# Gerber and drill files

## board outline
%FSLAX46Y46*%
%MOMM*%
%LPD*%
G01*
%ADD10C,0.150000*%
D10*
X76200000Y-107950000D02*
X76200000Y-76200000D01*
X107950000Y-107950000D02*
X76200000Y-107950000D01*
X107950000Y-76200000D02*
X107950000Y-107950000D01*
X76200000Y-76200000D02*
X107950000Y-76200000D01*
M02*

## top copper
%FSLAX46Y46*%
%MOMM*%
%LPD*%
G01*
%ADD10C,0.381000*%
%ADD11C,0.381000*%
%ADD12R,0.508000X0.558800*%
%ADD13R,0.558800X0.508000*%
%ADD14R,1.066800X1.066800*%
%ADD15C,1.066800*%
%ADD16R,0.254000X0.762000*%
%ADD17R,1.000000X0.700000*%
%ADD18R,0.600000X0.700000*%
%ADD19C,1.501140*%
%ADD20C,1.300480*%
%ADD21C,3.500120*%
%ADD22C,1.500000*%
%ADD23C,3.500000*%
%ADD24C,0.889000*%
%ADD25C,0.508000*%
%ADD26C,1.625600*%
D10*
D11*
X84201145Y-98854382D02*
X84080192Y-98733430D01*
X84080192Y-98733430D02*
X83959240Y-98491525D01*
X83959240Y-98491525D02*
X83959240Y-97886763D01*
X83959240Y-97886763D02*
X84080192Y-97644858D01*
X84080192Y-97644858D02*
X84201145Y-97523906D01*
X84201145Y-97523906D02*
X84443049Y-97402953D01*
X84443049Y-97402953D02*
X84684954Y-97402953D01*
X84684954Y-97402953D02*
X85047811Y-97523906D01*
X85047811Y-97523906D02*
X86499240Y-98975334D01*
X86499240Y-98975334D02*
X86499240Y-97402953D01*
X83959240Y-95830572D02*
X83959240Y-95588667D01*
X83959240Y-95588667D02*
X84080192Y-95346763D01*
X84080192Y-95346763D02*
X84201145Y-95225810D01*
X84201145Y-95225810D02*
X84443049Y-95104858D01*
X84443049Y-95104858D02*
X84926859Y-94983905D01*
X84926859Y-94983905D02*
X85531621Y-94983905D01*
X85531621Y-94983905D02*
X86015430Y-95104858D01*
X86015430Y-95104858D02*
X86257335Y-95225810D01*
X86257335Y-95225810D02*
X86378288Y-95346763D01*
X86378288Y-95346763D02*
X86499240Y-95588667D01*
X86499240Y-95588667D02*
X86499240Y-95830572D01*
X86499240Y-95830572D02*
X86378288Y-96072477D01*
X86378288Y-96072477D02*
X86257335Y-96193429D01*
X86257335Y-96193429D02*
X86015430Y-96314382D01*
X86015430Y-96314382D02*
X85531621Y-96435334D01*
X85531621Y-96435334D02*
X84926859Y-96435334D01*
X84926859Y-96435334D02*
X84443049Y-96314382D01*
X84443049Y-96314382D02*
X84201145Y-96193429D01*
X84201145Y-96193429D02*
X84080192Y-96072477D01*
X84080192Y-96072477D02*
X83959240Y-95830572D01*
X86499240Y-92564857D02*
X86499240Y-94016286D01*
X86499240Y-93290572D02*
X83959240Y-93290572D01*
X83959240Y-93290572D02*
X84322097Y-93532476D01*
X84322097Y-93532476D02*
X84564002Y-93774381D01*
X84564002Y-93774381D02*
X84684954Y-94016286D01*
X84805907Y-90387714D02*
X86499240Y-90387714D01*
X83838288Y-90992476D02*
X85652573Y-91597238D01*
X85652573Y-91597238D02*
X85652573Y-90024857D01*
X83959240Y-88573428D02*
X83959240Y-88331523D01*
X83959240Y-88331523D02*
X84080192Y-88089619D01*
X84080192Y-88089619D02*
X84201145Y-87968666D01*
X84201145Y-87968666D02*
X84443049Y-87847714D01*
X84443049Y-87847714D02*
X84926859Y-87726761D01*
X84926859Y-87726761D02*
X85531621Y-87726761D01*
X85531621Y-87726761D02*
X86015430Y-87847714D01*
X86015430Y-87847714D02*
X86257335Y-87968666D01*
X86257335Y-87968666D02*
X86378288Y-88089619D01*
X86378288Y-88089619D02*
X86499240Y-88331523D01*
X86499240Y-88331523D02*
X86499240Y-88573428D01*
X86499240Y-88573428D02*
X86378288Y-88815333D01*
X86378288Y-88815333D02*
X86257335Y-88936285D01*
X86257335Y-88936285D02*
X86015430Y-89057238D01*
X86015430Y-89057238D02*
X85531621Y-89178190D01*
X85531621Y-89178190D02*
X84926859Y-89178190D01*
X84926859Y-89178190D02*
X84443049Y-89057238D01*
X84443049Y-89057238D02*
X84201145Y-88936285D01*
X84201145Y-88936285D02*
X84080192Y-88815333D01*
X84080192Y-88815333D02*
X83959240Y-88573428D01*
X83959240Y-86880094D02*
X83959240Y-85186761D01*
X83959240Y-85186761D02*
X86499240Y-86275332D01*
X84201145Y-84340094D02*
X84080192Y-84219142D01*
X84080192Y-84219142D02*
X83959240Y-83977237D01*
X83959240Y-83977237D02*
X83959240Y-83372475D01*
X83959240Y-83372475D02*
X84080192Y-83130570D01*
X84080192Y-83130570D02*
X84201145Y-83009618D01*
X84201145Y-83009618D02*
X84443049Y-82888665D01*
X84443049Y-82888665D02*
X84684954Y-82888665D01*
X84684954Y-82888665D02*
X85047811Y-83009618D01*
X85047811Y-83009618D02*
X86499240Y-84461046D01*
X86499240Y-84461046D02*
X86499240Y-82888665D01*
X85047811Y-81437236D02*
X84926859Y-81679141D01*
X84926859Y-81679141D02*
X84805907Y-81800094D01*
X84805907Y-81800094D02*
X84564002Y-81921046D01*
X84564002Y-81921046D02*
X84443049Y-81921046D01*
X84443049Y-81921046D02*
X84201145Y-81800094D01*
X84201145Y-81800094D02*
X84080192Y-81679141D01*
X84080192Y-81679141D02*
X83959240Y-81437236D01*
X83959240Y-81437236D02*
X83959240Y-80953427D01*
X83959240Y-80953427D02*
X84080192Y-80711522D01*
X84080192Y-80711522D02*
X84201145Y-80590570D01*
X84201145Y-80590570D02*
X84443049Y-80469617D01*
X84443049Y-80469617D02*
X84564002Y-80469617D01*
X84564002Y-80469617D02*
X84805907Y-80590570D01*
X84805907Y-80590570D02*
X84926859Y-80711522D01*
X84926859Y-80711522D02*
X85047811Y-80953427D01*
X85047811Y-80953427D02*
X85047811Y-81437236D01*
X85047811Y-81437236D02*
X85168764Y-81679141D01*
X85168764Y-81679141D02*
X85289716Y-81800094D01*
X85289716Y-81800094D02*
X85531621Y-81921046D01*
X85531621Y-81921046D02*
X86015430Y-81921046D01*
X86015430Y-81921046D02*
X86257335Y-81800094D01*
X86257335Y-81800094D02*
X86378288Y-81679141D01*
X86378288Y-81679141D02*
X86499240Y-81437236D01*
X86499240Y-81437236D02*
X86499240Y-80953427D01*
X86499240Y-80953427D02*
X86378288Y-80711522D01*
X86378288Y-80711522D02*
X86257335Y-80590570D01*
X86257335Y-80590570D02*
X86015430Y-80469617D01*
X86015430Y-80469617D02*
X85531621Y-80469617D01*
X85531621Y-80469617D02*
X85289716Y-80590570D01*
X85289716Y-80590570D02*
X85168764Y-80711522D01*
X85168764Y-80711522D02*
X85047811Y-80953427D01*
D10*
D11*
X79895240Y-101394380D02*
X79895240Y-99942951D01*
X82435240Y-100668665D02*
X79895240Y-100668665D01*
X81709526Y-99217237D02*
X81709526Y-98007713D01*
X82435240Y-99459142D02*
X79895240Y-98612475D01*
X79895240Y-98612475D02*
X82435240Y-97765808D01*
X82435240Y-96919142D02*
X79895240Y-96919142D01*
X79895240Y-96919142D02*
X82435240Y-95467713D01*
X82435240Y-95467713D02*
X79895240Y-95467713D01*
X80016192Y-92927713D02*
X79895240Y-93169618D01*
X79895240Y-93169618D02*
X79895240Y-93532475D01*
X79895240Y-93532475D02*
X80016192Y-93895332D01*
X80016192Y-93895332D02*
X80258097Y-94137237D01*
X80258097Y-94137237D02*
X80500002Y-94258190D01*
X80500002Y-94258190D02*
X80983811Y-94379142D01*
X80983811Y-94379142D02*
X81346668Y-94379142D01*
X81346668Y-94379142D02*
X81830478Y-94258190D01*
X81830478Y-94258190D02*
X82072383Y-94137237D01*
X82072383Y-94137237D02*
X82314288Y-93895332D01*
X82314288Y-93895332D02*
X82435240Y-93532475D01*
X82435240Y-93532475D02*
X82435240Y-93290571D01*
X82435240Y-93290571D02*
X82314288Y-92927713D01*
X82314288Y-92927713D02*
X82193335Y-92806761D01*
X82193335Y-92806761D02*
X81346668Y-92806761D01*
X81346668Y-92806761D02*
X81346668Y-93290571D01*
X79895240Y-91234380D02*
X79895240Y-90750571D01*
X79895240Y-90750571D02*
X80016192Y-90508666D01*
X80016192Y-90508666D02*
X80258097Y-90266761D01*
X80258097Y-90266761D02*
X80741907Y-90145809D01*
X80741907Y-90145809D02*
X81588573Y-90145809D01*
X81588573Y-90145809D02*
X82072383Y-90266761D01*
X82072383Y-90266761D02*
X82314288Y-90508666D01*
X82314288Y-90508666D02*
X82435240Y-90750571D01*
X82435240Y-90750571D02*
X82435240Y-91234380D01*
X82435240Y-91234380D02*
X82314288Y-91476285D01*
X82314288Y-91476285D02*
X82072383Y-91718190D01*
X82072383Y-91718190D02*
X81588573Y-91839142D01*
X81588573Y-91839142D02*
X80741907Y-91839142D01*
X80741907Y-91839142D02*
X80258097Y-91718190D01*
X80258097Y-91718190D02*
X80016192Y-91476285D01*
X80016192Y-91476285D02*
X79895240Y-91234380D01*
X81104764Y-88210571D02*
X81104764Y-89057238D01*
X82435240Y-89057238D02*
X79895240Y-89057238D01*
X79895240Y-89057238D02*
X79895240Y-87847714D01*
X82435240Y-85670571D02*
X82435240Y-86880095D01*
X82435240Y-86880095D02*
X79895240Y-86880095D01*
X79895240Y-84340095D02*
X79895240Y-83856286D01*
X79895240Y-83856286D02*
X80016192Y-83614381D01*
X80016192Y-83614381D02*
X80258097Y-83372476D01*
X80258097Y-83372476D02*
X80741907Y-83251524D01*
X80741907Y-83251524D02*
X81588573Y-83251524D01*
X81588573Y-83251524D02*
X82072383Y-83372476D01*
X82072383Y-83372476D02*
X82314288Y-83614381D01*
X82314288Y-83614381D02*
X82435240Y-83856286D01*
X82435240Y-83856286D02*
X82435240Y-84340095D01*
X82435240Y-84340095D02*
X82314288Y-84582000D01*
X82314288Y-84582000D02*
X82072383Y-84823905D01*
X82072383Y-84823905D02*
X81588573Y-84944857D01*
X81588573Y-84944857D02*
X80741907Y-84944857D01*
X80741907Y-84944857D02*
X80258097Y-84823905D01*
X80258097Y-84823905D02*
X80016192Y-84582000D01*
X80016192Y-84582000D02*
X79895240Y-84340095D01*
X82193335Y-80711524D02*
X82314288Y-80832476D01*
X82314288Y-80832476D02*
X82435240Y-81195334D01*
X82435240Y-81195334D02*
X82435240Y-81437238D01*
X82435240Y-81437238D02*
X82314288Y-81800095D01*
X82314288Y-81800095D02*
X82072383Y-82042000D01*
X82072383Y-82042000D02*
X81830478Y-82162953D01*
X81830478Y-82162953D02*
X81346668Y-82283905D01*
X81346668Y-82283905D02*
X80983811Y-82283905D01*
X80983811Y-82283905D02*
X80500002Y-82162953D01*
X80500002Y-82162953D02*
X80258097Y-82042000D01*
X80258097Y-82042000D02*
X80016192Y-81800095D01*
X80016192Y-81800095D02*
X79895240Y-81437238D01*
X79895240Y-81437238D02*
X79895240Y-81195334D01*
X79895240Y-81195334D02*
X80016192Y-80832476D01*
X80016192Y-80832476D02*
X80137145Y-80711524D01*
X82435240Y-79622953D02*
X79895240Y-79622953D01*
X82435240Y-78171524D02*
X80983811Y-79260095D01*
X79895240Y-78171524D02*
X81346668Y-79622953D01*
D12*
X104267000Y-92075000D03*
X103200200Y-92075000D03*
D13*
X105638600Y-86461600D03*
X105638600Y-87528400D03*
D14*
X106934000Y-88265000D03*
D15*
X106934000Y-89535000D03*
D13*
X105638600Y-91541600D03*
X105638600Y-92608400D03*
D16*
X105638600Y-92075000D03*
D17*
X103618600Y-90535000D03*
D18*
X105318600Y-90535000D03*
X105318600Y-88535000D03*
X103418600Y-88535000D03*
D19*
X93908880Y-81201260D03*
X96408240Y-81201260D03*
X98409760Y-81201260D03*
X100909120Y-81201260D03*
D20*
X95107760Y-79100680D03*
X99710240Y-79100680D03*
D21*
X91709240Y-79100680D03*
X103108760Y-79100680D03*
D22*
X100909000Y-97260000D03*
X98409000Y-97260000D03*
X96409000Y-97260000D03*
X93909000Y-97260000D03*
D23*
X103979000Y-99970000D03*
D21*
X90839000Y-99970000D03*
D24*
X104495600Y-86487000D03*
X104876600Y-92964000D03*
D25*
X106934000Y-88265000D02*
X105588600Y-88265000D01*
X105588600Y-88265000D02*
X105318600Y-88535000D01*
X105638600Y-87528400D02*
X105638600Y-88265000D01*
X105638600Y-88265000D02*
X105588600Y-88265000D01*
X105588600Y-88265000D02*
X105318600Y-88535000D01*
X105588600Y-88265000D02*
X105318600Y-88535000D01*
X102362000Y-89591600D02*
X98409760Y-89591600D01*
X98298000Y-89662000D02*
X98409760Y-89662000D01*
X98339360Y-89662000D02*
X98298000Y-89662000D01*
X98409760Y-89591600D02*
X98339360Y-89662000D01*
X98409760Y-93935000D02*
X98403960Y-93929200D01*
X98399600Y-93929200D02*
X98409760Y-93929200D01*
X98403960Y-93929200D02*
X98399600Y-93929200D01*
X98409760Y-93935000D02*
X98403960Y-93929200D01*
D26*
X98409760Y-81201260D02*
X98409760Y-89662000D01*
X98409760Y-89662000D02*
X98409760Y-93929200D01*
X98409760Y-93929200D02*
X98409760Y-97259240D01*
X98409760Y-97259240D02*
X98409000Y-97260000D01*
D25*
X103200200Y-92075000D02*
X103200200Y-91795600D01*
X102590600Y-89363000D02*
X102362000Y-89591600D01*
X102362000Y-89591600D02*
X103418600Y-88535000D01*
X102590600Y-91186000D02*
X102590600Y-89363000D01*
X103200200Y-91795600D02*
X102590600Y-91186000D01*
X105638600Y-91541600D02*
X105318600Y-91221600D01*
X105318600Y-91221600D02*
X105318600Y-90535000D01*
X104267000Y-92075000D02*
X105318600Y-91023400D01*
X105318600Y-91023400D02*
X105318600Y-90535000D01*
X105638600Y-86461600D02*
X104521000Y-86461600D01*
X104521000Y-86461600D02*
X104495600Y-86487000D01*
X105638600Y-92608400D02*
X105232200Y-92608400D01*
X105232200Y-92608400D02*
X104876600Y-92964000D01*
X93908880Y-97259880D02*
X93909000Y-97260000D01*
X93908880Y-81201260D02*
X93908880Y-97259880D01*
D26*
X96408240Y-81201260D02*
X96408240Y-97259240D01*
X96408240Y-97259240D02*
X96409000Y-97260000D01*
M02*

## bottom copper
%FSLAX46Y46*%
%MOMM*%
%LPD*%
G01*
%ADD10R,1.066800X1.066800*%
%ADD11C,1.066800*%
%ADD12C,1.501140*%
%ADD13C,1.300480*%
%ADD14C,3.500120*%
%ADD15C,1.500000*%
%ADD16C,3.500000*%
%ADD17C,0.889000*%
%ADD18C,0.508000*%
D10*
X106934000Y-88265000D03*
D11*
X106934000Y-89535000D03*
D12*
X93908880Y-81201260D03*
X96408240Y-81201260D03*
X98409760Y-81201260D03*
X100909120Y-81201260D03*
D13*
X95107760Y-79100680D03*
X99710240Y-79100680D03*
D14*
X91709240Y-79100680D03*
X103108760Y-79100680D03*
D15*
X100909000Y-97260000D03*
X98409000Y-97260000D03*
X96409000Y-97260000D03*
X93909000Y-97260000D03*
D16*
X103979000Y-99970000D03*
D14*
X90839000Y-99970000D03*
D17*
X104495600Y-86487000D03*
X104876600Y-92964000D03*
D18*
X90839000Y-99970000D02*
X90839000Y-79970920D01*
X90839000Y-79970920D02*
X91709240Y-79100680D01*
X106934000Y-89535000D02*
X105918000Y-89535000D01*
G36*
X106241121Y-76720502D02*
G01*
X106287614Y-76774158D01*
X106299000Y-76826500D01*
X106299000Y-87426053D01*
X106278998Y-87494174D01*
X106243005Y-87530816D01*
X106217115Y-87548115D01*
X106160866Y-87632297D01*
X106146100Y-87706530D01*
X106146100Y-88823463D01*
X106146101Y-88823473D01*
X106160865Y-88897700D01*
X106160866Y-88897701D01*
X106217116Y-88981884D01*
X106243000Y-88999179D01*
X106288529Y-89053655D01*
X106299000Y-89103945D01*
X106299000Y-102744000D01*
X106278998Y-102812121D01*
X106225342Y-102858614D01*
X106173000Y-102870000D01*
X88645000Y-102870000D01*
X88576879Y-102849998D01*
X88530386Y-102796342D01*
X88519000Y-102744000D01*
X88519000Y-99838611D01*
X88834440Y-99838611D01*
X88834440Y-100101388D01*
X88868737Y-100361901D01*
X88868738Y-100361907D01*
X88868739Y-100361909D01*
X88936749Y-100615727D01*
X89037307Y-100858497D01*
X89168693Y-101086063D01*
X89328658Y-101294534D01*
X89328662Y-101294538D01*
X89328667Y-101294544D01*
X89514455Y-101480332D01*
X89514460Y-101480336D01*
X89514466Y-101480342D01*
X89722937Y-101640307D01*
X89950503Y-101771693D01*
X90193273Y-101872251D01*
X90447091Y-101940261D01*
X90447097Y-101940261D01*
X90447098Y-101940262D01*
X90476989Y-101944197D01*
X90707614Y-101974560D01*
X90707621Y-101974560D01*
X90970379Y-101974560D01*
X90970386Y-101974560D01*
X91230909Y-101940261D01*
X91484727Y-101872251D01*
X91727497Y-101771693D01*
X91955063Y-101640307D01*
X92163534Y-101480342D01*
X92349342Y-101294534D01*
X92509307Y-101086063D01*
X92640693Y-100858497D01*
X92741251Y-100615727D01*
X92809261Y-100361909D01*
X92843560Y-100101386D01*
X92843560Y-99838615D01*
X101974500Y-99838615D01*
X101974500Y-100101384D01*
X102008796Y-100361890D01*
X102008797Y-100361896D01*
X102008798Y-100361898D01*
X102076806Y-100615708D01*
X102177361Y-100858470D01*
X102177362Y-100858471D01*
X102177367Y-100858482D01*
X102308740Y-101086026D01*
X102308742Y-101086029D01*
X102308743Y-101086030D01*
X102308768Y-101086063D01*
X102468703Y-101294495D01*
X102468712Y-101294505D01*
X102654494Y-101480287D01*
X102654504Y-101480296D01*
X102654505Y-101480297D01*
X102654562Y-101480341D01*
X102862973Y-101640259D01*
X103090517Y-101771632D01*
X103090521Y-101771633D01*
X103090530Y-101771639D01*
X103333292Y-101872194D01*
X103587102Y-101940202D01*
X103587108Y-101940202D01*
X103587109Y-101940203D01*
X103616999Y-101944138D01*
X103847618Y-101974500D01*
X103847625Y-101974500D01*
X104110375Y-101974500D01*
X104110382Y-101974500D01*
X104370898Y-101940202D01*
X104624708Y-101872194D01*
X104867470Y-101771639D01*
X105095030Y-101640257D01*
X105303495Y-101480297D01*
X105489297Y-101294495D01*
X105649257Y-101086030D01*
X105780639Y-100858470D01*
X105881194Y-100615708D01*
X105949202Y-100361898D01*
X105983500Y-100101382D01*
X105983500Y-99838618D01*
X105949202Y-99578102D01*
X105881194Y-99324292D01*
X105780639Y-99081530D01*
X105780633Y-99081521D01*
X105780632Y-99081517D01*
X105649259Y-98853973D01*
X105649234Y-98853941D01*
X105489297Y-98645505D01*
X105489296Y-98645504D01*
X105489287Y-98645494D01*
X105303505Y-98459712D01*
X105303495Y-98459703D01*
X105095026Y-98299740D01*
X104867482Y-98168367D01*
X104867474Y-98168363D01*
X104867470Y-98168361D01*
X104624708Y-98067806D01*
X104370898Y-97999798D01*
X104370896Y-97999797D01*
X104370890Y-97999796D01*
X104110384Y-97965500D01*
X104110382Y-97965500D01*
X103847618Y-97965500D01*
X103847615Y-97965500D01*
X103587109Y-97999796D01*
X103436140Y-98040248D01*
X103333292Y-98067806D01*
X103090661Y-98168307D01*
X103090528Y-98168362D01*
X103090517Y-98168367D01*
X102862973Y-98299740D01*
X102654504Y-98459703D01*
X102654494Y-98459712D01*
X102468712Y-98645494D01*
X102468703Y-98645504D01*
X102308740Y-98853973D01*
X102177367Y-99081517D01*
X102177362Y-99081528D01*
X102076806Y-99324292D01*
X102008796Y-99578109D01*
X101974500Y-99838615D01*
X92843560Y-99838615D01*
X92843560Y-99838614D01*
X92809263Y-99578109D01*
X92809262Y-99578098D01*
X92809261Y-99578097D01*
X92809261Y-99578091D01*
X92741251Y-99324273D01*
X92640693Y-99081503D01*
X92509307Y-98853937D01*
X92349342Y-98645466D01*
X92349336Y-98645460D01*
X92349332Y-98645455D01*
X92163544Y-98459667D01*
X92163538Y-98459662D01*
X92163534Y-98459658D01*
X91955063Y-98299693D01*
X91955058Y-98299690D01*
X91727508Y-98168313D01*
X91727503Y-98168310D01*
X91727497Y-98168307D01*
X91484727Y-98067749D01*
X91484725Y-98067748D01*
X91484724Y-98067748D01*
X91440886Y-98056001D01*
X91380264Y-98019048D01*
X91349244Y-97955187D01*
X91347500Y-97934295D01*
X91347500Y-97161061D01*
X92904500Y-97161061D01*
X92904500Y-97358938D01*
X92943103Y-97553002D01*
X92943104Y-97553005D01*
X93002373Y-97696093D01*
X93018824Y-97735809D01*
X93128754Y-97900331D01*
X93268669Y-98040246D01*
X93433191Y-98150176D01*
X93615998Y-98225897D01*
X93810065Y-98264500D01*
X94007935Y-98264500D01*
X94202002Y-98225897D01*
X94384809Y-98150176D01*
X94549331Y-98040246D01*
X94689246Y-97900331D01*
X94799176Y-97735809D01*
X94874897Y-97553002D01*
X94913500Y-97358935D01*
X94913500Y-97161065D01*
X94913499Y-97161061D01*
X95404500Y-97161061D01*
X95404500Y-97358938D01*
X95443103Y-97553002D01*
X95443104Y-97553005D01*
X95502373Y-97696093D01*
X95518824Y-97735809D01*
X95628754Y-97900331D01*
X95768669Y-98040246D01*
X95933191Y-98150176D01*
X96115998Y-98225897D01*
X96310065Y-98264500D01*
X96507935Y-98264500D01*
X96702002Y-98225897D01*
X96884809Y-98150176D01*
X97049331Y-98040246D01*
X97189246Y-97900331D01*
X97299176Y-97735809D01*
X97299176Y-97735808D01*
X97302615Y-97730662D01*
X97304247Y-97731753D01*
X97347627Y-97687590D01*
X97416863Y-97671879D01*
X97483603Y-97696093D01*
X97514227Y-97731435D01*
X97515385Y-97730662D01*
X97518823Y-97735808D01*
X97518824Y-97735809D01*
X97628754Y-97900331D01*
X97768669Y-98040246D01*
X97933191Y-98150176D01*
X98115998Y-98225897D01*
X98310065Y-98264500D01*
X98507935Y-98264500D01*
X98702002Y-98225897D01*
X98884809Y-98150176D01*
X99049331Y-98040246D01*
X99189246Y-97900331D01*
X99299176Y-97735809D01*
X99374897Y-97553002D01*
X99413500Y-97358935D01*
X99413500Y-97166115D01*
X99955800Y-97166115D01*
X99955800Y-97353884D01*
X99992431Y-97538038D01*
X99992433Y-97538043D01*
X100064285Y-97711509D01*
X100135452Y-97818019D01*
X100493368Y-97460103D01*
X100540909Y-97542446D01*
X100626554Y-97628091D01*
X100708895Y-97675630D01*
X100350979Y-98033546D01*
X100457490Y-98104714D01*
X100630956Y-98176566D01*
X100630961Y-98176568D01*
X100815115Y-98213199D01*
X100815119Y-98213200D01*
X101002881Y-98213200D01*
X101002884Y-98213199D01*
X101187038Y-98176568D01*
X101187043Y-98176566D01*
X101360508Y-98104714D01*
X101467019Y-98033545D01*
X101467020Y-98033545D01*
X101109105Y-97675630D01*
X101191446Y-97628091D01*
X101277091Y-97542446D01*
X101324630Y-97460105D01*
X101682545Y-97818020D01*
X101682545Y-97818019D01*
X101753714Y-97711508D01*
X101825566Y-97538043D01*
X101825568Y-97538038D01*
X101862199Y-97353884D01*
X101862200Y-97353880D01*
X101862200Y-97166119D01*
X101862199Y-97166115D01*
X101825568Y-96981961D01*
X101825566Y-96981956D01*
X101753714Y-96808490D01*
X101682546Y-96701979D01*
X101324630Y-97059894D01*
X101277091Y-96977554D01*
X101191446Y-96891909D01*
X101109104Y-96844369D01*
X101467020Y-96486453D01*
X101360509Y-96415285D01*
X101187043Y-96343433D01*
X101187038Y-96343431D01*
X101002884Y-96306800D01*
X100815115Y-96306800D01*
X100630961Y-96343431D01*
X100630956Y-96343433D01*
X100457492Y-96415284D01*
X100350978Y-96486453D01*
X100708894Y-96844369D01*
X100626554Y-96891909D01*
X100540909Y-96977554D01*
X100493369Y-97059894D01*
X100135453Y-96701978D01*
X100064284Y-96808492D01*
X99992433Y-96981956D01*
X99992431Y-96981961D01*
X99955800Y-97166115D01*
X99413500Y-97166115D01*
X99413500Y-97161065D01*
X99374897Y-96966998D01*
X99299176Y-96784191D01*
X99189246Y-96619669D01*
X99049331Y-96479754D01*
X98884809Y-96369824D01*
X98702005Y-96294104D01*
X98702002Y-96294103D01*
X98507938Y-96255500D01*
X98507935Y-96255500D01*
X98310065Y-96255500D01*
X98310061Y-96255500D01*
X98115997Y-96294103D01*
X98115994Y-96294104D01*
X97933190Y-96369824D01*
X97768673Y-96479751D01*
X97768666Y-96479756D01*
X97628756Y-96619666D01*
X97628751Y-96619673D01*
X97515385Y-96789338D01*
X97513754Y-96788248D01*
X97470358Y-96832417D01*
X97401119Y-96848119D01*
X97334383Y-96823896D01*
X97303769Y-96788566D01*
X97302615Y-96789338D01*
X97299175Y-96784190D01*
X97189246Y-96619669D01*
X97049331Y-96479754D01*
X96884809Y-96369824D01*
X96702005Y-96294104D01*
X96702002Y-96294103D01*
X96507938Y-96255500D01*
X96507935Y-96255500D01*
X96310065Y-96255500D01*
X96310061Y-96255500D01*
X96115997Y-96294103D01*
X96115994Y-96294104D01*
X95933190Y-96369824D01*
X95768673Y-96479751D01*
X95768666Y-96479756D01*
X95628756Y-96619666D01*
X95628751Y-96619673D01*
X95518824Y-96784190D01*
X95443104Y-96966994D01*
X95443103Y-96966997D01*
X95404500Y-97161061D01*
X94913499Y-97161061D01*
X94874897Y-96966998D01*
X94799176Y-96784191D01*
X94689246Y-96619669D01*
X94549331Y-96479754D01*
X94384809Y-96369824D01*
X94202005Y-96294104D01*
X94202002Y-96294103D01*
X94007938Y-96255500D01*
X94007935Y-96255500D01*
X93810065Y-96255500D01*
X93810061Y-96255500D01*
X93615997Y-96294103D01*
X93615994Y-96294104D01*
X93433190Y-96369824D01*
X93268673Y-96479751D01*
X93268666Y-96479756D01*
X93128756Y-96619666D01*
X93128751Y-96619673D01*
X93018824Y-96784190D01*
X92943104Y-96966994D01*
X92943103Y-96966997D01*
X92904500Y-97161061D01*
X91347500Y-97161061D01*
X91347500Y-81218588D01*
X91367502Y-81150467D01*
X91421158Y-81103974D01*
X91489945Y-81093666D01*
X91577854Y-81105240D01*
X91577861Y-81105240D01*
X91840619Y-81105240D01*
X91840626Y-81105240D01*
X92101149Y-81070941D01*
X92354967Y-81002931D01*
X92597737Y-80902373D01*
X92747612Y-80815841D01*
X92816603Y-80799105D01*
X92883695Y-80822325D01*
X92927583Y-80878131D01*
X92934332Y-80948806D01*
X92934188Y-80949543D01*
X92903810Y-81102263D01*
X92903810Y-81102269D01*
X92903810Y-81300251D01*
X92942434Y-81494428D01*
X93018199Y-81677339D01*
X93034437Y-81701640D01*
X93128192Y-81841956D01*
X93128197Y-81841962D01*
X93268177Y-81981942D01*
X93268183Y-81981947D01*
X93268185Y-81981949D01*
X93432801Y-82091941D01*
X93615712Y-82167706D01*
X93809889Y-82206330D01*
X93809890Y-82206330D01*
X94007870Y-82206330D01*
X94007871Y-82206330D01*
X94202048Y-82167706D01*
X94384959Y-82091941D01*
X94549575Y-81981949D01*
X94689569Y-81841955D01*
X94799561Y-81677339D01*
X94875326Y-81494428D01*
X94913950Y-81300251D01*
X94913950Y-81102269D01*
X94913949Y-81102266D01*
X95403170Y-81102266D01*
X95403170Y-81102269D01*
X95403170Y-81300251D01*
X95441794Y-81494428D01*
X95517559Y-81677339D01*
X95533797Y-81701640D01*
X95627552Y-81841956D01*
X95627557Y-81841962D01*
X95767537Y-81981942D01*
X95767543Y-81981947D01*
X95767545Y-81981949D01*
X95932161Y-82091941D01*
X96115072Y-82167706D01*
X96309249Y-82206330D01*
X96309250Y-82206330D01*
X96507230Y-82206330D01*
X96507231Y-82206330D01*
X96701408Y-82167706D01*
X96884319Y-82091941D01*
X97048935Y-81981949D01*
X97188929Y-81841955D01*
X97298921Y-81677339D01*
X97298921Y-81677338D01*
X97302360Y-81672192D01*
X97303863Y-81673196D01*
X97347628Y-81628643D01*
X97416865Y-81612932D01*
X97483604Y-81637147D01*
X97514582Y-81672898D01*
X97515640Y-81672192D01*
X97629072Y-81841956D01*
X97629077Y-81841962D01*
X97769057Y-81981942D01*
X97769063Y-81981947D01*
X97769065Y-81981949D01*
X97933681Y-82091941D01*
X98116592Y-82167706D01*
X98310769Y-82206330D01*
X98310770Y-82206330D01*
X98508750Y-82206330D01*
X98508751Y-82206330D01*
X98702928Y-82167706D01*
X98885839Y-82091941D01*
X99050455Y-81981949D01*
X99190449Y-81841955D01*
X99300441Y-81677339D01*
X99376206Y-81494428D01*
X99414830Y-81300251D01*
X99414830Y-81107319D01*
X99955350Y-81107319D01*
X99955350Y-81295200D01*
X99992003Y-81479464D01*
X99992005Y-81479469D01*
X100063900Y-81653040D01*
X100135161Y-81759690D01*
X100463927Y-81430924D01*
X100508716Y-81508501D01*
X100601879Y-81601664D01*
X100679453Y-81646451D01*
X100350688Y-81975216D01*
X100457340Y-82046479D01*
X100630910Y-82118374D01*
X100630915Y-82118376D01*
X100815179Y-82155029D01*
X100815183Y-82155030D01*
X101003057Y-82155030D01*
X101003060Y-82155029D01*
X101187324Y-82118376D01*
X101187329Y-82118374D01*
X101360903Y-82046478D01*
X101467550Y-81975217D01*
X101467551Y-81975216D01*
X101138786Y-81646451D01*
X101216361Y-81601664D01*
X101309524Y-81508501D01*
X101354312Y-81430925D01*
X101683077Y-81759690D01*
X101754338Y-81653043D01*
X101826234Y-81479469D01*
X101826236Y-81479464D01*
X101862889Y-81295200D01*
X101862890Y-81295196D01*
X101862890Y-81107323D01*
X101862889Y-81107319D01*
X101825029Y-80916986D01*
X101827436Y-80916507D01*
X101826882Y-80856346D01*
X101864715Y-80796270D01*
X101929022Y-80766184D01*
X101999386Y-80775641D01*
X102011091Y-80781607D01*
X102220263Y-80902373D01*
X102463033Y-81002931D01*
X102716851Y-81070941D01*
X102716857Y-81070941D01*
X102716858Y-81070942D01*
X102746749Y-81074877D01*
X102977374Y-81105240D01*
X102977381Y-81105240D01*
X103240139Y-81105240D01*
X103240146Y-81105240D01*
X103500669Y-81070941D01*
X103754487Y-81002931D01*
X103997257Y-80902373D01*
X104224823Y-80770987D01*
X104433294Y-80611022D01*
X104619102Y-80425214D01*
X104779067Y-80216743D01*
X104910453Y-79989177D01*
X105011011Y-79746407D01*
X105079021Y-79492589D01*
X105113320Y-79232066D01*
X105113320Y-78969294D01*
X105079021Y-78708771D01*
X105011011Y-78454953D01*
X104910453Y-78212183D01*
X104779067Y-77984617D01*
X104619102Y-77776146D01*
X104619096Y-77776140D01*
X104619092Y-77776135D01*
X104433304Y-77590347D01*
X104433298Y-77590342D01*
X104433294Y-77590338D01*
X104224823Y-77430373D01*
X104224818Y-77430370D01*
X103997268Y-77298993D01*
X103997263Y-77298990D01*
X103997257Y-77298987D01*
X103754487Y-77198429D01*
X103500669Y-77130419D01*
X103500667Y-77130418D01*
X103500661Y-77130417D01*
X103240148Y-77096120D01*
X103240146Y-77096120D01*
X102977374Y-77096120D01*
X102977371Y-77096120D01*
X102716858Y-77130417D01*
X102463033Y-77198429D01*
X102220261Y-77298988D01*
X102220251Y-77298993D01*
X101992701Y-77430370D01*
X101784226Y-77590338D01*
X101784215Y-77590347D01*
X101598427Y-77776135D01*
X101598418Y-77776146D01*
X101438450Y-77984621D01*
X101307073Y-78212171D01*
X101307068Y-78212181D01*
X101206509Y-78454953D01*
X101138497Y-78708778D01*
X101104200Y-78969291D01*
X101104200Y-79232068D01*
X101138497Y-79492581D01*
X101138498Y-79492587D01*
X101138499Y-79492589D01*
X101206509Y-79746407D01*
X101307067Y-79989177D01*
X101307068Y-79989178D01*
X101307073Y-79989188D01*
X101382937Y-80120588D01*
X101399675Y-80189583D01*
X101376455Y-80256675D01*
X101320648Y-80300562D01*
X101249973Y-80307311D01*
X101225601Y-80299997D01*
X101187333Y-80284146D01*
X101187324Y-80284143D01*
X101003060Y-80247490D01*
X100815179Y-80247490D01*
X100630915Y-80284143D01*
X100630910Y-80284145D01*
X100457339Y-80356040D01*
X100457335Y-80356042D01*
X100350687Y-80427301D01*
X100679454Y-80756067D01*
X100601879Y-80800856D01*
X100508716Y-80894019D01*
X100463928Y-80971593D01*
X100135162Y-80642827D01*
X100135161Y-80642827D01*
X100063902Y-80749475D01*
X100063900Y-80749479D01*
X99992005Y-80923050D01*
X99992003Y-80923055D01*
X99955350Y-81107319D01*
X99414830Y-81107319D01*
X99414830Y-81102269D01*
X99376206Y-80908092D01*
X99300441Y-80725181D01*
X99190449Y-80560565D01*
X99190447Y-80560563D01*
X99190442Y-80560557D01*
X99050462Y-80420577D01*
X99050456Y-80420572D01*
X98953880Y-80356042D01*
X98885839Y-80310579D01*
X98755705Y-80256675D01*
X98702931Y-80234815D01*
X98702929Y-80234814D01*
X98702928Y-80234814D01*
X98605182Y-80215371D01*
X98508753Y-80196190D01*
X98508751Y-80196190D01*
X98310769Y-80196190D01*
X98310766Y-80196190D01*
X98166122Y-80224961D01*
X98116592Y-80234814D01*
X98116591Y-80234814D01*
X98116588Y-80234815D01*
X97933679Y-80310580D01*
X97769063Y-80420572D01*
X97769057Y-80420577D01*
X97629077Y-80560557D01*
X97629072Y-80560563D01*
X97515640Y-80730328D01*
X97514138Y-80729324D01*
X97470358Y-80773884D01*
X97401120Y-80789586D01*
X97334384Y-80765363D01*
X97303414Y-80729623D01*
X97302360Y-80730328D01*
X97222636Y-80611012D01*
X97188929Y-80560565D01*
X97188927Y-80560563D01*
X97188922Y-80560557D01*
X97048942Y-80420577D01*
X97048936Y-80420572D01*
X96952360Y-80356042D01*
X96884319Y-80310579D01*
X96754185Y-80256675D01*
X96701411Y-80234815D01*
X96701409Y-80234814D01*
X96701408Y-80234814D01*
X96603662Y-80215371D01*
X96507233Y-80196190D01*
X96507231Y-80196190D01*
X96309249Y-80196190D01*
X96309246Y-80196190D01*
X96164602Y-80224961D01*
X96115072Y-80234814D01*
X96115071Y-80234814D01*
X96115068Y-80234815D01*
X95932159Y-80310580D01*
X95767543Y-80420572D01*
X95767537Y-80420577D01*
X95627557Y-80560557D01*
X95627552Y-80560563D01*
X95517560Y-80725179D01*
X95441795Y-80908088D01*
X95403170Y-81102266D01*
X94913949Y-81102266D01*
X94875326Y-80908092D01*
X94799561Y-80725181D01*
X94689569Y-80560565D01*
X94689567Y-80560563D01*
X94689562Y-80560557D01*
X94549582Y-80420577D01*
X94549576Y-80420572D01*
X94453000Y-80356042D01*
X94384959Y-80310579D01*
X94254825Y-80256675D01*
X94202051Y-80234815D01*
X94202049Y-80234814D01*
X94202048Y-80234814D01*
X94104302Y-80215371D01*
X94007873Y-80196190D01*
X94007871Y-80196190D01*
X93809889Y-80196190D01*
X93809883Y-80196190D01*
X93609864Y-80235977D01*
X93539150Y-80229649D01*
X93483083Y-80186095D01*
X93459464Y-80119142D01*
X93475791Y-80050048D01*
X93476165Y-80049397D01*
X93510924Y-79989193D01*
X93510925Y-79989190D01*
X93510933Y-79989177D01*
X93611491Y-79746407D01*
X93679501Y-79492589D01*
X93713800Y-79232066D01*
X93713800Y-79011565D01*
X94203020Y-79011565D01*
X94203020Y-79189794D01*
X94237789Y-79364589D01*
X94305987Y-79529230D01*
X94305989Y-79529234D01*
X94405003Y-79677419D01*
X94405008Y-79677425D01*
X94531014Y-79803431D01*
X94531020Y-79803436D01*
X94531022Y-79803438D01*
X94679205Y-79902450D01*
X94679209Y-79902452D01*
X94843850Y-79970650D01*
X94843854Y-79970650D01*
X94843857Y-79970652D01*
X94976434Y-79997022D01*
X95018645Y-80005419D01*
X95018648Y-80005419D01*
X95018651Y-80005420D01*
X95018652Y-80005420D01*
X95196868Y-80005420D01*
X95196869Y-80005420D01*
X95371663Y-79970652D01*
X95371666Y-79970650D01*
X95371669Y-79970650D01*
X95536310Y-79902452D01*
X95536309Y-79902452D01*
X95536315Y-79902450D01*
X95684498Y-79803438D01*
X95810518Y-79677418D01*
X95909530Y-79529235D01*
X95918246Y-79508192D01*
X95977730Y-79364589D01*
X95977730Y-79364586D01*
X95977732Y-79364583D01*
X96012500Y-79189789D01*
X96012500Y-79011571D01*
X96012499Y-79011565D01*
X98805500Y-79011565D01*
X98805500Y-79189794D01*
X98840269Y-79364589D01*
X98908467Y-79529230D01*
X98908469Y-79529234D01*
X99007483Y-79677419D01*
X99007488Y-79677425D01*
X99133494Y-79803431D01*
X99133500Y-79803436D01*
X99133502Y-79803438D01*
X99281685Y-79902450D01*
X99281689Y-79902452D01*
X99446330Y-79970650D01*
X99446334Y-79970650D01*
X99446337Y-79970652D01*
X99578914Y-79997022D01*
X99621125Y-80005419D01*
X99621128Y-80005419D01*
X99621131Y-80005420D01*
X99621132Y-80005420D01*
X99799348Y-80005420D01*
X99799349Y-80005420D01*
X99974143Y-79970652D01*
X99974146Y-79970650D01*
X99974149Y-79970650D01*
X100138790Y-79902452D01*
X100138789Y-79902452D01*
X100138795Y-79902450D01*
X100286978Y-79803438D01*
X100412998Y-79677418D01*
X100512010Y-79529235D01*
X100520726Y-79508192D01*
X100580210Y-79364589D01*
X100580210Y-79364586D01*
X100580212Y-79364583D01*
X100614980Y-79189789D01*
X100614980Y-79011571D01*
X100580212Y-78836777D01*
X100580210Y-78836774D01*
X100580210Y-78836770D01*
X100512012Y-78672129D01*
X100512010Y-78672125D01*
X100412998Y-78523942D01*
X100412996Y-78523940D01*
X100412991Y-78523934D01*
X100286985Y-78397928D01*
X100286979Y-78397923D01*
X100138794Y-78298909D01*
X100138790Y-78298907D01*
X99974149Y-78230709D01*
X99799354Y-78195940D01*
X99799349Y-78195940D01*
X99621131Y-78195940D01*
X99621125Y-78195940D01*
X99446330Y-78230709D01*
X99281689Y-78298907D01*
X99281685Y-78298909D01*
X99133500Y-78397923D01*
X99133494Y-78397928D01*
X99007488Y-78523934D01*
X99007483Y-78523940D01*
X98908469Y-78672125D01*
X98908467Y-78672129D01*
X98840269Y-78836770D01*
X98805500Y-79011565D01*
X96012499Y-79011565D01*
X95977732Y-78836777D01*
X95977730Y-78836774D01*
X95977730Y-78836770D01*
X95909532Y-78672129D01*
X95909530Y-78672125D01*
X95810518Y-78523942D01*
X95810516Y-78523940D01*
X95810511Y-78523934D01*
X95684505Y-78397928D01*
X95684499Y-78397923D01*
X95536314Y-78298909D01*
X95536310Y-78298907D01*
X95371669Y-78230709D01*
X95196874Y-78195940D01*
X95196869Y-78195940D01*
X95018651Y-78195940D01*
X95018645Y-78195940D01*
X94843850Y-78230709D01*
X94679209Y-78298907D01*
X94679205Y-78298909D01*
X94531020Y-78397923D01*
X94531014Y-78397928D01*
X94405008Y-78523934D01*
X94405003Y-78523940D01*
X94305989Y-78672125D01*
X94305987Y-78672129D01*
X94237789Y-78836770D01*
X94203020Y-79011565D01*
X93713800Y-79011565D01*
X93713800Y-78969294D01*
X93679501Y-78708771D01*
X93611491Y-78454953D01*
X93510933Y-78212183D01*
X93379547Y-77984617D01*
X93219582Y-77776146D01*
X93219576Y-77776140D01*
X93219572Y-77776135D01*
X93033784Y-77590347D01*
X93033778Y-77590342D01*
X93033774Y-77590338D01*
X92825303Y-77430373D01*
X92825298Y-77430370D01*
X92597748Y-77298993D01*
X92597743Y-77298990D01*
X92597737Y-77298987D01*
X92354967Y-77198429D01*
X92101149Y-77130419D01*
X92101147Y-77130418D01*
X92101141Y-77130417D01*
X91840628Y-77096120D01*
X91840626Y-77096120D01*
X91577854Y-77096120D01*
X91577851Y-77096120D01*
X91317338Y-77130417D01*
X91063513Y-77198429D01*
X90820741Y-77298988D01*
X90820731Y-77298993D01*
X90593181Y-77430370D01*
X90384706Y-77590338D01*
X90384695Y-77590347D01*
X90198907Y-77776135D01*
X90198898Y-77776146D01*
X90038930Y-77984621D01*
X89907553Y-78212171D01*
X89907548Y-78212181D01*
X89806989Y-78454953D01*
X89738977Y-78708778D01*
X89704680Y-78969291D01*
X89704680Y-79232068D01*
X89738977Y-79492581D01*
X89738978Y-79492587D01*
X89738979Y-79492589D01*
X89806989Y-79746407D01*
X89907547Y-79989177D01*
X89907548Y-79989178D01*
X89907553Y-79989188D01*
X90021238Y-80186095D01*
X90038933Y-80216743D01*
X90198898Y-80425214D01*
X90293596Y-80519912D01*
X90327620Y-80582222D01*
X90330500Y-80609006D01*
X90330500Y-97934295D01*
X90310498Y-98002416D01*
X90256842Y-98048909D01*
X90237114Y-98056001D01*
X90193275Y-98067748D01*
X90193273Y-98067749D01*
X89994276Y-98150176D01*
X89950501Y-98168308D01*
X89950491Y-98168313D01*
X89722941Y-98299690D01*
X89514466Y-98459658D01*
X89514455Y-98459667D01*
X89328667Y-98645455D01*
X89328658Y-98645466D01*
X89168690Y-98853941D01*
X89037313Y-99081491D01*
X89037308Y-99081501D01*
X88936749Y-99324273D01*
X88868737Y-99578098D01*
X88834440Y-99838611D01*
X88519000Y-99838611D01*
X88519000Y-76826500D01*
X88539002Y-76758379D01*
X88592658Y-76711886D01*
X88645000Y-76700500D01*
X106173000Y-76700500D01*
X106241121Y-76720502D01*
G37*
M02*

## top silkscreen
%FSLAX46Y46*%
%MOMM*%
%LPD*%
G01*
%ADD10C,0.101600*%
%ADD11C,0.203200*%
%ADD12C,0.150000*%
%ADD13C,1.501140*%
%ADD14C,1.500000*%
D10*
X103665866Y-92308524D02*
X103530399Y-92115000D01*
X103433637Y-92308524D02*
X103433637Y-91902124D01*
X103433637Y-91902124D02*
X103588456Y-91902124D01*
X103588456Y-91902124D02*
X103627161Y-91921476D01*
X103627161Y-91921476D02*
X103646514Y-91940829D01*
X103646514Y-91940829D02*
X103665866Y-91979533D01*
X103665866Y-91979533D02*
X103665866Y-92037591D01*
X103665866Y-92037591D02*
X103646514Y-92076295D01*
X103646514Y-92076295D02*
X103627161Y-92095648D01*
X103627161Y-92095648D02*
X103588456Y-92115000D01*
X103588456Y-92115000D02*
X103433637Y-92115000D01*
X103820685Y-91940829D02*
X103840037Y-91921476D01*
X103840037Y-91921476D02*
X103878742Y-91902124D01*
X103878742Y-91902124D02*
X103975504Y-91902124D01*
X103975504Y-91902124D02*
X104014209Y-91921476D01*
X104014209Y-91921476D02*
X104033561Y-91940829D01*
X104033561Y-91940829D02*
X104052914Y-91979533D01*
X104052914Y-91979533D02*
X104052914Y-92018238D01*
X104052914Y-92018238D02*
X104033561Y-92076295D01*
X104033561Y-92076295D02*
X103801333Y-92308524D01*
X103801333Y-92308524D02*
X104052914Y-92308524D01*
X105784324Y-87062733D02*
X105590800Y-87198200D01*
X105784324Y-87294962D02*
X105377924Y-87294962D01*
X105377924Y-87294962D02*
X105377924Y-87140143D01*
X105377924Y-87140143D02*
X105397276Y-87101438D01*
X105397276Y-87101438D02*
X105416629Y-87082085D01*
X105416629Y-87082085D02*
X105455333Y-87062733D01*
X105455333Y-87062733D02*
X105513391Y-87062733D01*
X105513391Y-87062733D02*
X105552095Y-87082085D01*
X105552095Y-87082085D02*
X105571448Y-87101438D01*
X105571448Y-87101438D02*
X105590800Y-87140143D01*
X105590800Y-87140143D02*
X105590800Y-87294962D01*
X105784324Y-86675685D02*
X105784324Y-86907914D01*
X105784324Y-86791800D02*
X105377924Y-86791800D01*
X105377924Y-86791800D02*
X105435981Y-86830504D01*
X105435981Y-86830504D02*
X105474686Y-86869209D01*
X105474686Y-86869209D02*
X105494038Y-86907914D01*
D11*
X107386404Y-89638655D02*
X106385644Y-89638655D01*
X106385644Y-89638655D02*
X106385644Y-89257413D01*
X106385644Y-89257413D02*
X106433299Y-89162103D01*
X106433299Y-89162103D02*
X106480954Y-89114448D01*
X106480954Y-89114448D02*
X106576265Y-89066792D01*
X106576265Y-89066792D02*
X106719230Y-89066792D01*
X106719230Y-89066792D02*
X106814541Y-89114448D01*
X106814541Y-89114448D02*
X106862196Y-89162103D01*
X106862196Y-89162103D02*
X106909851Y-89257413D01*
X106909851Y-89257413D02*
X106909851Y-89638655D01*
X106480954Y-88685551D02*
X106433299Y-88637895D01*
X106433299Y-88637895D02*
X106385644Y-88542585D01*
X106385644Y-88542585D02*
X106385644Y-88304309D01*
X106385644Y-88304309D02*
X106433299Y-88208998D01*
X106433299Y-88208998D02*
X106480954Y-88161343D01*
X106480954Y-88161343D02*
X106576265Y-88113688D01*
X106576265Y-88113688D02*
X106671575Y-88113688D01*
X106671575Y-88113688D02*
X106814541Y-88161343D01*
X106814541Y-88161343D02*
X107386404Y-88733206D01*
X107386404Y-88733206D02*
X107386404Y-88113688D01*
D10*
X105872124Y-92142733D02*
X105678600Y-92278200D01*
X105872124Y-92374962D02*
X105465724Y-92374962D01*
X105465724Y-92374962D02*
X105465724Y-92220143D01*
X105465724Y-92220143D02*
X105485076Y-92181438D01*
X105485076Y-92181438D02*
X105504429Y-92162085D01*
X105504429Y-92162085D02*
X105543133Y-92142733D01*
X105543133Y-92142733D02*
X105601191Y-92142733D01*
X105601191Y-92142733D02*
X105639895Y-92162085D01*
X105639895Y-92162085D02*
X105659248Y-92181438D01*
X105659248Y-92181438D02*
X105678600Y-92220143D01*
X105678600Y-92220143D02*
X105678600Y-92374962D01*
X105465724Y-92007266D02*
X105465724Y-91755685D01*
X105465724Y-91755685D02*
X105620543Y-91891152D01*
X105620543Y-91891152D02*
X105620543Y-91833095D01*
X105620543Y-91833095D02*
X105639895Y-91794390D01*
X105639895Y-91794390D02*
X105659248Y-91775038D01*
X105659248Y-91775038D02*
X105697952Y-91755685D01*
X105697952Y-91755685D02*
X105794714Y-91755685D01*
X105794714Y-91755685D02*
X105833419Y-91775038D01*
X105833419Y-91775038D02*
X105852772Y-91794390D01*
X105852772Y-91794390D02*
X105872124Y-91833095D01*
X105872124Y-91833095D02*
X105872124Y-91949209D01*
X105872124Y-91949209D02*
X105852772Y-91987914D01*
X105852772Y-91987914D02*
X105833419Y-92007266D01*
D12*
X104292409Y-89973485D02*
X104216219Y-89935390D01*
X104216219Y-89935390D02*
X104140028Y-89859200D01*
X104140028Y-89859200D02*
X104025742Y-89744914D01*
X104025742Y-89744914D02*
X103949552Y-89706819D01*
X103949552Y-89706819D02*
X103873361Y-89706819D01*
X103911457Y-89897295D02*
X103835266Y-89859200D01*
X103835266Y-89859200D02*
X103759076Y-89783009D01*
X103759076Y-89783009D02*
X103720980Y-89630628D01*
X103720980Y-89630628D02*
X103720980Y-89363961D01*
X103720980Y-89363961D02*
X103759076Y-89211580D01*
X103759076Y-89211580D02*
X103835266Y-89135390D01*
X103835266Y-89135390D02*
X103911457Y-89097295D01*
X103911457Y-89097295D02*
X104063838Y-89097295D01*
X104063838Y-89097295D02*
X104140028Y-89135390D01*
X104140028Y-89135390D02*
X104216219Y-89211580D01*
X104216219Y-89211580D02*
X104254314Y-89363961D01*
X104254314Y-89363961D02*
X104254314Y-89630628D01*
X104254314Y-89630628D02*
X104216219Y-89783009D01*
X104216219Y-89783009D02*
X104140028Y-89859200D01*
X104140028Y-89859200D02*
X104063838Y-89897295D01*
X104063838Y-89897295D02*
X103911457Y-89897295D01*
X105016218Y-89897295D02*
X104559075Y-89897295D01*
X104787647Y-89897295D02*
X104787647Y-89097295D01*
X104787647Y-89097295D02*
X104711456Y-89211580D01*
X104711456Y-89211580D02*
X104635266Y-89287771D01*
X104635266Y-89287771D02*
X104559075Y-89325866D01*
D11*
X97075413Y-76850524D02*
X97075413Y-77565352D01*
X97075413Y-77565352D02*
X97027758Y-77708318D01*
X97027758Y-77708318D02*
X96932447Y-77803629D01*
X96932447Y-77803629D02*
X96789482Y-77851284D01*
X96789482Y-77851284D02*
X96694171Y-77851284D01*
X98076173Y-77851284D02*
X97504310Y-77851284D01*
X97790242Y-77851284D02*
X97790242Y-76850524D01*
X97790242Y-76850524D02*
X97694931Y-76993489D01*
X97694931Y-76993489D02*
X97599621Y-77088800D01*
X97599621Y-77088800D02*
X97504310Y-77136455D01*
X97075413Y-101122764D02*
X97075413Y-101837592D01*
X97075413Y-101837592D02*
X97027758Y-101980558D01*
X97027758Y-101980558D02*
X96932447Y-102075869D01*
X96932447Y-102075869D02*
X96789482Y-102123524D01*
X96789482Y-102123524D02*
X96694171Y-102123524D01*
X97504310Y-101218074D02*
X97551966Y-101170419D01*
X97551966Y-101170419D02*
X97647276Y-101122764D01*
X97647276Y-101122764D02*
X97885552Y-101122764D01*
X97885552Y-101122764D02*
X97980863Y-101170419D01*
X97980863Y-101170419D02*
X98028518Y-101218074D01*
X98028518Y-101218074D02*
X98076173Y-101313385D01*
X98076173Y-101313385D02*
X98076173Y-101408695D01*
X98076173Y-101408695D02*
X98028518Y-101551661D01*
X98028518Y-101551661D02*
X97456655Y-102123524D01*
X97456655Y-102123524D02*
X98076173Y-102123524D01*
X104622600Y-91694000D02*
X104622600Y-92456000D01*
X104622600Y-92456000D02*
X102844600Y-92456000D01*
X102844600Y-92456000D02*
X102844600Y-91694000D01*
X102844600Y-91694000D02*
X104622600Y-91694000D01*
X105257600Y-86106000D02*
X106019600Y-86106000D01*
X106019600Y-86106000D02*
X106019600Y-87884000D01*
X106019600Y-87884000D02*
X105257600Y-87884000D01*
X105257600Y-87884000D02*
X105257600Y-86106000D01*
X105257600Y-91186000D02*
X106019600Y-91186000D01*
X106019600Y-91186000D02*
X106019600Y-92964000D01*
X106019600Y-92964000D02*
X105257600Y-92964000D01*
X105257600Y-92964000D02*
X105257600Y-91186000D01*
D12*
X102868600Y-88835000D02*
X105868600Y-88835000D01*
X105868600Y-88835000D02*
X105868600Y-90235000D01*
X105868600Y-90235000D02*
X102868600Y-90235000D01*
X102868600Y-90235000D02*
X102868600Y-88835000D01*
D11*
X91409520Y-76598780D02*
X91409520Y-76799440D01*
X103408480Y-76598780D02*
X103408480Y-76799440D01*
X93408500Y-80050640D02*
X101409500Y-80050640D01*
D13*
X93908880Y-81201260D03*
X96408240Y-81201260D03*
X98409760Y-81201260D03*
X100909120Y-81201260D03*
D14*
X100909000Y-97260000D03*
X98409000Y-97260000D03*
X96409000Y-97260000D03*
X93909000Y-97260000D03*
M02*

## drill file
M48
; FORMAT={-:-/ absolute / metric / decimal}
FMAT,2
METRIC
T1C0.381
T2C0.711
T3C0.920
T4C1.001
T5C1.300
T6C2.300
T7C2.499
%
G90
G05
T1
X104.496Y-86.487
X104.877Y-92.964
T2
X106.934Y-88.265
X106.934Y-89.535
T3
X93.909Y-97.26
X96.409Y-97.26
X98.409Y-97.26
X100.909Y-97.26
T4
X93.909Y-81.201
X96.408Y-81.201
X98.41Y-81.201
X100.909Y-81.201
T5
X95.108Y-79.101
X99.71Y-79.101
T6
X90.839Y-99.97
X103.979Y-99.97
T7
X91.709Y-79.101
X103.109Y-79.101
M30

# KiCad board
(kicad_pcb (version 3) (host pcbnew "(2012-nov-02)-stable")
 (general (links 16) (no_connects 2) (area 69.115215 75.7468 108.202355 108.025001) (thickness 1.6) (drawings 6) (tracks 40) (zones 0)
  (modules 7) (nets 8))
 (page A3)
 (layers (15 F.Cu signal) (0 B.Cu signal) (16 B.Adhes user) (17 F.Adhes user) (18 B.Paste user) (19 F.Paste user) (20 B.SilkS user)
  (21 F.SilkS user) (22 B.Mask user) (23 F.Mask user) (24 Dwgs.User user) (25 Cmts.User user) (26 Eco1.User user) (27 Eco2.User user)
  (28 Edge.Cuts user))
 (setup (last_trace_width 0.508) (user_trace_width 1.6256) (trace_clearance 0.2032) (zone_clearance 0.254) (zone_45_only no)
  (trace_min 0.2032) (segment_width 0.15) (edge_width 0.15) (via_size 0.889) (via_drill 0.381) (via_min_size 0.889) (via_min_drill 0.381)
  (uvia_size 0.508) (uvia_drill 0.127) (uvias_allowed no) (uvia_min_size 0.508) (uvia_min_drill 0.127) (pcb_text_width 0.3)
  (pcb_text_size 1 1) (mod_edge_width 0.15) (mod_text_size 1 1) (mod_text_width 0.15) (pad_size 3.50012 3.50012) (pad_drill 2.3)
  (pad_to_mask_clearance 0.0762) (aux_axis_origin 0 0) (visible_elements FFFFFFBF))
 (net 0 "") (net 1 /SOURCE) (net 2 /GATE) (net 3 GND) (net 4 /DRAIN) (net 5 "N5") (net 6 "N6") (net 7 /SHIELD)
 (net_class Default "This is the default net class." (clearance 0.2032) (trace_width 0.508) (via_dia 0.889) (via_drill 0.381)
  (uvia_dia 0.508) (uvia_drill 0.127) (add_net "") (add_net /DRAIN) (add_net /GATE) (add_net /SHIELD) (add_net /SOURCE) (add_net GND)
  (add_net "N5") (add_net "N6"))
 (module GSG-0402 (layer F.Cu) (at 103.7336 92.075) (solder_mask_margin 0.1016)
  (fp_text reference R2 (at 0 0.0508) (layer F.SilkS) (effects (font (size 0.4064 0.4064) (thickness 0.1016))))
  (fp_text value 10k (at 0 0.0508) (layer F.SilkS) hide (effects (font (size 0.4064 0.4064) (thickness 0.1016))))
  (fp_line (start 0.889 -0.381) (end 0.889 0.381) (layer F.SilkS) (width 0.2032))
  (fp_line (start 0.889 0.381) (end -0.889 0.381) (layer F.SilkS) (width 0.2032))
  (fp_line (start -0.889 0.381) (end -0.889 -0.381) (layer F.SilkS) (width 0.2032))
  (fp_line (start -0.889 -0.381) (end 0.889 -0.381) (layer F.SilkS) (width 0.2032))
  (pad 2 smd rect (at 0.5334 0) (size 0.508 0.5588) (layers F.Cu F.Paste F.Mask) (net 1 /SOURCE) (solder_mask_margin 0.1016))
  (pad 1 smd rect (at -0.5334 0) (size 0.508 0.5588) (layers F.Cu F.Paste F.Mask) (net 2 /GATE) (die_length -2147.483648)
   (solder_mask_margin 0.1016)))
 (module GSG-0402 (layer F.Cu) (at 105.6386 86.995 90) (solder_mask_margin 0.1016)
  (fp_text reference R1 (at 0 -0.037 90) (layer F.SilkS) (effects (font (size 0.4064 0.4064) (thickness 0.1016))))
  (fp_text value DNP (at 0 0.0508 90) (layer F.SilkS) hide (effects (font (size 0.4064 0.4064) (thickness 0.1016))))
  (fp_line (start 0.889 -0.381) (end 0.889 0.381) (layer F.SilkS) (width 0.2032))
  (fp_line (start 0.889 0.381) (end -0.889 0.381) (layer F.SilkS) (width 0.2032))
  (fp_line (start -0.889 0.381) (end -0.889 -0.381) (layer F.SilkS) (width 0.2032))
  (fp_line (start -0.889 -0.381) (end 0.889 -0.381) (layer F.SilkS) (width 0.2032))
  (pad 2 smd rect (at 0.5334 0 90) (size 0.508 0.5588) (layers F.Cu F.Paste F.Mask) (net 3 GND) (solder_mask_margin 0.1016))
  (pad 1 smd rect (at -0.5334 0 90) (size 0.508 0.5588) (layers F.Cu F.Paste F.Mask) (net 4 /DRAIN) (die_length -2147.483648)
   (solder_mask_margin 0.1016)))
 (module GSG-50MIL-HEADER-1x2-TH (layer F.Cu) (at 106.934 88.9 270)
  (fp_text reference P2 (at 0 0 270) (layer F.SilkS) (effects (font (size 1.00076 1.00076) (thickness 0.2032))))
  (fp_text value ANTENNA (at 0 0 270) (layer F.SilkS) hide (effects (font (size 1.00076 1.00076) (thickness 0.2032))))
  (pad 1 thru_hole rect (at -0.635 0 270) (size 1.0668 1.0668) (drill 0.7112) (layers *.Cu *.Mask) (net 4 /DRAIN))
  (pad 2 thru_hole circle (at 0.635 0 270) (size 1.0668 1.0668) (drill 0.7112) (layers *.Cu *.Mask) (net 3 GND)))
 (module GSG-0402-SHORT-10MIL (layer F.Cu) (at 105.6386 92.075 90) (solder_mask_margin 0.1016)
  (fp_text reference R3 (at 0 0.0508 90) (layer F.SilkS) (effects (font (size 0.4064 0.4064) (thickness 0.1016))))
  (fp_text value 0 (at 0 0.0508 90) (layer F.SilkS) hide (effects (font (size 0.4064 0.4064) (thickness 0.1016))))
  (fp_line (start 0.889 -0.381) (end 0.889 0.381) (layer F.SilkS) (width 0.2032))
  (fp_line (start 0.889 0.381) (end -0.889 0.381) (layer F.SilkS) (width 0.2032))
  (fp_line (start -0.889 0.381) (end -0.889 -0.381) (layer F.SilkS) (width 0.2032))
  (fp_line (start -0.889 -0.381) (end 0.889 -0.381) (layer F.SilkS) (width 0.2032))
  (pad 2 smd rect (at 0.5334 0 90) (size 0.508 0.5588) (layers F.Cu F.Mask) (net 1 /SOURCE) (solder_mask_margin 0.1016))
  (pad 1 smd rect (at -0.5334 0 90) (size 0.508 0.5588) (layers F.Cu F.Mask) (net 3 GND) (die_length -2147.483648)
   (solder_mask_margin 0.1016))
  (pad "" smd rect (at 0 0 90) (size 0.762 0.254) (layers F.Cu F.Mask)))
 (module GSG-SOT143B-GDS (layer F.Cu) (at 104.3686 89.535)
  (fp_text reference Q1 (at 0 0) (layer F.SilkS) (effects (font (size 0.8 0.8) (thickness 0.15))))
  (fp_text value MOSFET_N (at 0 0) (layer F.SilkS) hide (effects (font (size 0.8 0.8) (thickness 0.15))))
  (fp_line (start -1.5 -0.7) (end 1.5 -0.7) (layer F.SilkS) (width 0.15))
  (fp_line (start 1.5 -0.7) (end 1.5 0.7) (layer F.SilkS) (width 0.15))
  (fp_line (start 1.5 0.7) (end -1.5 0.7) (layer F.SilkS) (width 0.15))
  (fp_line (start -1.5 0.7) (end -1.5 -0.7) (layer F.SilkS) (width 0.15))
  (pad B smd rect (at -0.75 1) (size 1 0.7) (layers F.Cu F.Paste F.Mask))
  (pad S smd rect (at 0.95 1) (size 0.6 0.7) (layers F.Cu F.Paste F.Mask) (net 1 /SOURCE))
  (pad D smd rect (at 0.95 -1) (size 0.6 0.7) (layers F.Cu F.Paste F.Mask) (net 4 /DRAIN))
  (pad G smd rect (at -0.95 -1) (size 0.6 0.7) (layers F.Cu F.Paste F.Mask) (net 2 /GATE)))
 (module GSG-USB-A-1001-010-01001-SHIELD (layer F.Cu) (at 97.409 76.2 180)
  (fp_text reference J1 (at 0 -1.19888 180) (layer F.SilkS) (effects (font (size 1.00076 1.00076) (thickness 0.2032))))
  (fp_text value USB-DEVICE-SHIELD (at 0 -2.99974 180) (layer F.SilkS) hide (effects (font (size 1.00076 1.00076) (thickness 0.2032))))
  (fp_line (start 5.99948 -0.39878) (end 5.99948 -0.59944) (layer F.SilkS) (width 0.2032))
  (fp_line (start -5.99948 -0.39878) (end -5.99948 -0.59944) (layer F.SilkS) (width 0.2032))
  (fp_line (start 4.0005 -3.85064) (end -4.0005 -3.85064) (layer F.SilkS) (width 0.2032))
  (pad 1 thru_hole circle (at 3.50012 -5.00126 180) (size 1.50114 1.50114) (drill 1.00076) (layers *.Cu *.Mask F.SilkS) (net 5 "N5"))
  (pad 2 thru_hole circle (at 1.00076 -5.00126 180) (size 1.50114 1.50114) (drill 1.00076) (layers *.Cu *.Mask F.SilkS) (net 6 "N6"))
  (pad 3 thru_hole circle (at -1.00076 -5.00126 180) (size 1.50114 1.50114) (drill 1.00076) (layers *.Cu *.Mask F.SilkS) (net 2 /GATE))
  (pad 4 thru_hole circle (at -3.50012 -5.00126 180) (size 1.50114 1.50114) (drill 1.00076) (layers *.Cu *.Mask F.SilkS) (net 3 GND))
  (pad "" thru_hole circle (at 2.30124 -2.90068 180) (size 1.30048 1.30048) (drill 1.30048) (layers *.Cu *.Mask) (clearance -0.09906))
  (pad "" thru_hole circle (at -2.30124 -2.90068 180) (size 1.30048 1.30048) (drill 1.30048) (layers *.Cu *.Mask) (clearance -0.09906))
  (pad 5 thru_hole circle (at 5.69976 -2.90068 180) (size 3.50012 3.50012) (drill 2.49936) (layers *.Cu *.Mask) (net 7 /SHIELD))
  (pad 5 thru_hole circle (at -5.69976 -2.90068 180) (size 3.50012 3.50012) (drill 2.49936) (layers *.Cu *.Mask) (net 7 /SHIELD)))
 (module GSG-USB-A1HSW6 (layer F.Cu) (at 97.409 102.87)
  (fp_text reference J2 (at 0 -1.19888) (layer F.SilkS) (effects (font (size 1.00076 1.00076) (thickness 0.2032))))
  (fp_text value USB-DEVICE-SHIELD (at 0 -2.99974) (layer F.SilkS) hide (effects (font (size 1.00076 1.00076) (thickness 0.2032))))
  (pad 4 thru_hole circle (at 3.5 -5.61) (size 1.5 1.5) (drill 0.92) (layers *.Cu *.Mask F.SilkS) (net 3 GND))
  (pad 3 thru_hole circle (at 1 -5.61) (size 1.5 1.5) (drill 0.92) (layers *.Cu *.Mask F.SilkS) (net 2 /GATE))
  (pad 2 thru_hole circle (at -1 -5.61) (size 1.5 1.5) (drill 0.92) (layers *.Cu *.Mask F.SilkS) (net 6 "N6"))
  (pad 1 thru_hole circle (at -3.5 -5.61) (size 1.5 1.5) (drill 0.92) (layers *.Cu *.Mask F.SilkS) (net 5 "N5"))
  (pad 5 thru_hole circle (at 6.57 -2.9) (size 3.5 3.5) (drill 2.3) (layers *.Cu *.Mask) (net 7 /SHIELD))
  (pad 5 thru_hole circle (at -6.57 -2.9) (size 3.50012 3.50012) (drill 2.3) (layers *.Cu *.Mask) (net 7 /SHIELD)))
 (gr_line (start 76.2 107.95) (end 76.2 76.2) (angle 90) (layer Edge.Cuts) (width 0.15))
 (gr_line (start 107.95 107.95) (end 76.2 107.95) (angle 90) (layer Edge.Cuts) (width 0.15))
 (gr_line (start 107.95 76.2) (end 107.95 107.95) (angle 90) (layer Edge.Cuts) (width 0.15))
 (gr_line (start 76.2 76.2) (end 107.95 76.2) (angle 90) (layer Edge.Cuts) (width 0.15))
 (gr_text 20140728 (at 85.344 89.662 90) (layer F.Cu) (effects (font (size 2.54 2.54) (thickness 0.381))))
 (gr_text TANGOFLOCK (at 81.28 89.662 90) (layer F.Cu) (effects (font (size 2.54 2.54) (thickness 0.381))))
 (segment (start 106.934 88.265) (end 105.5886 88.265) (width 0.508) (layer F.Cu) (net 4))
 (segment (start 105.5886 88.265) (end 105.3186 88.535) (width 0.508) (layer F.Cu) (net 4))
 (segment (start 105.6386 87.5284) (end 105.6386 88.265) (width 0.508) (layer F.Cu) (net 4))
 (segment (start 105.6386 88.265) (end 105.5886 88.265) (width 0.508) (layer F.Cu) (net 4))
 (segment (start 105.5886 88.265) (end 105.3186 88.535) (width 0.508) (layer F.Cu) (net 4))
 (segment (start 105.5886 88.265) (end 105.3186 88.535) (width 0.508) (layer F.Cu) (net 4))
 (segment (start 102.362 89.5916) (end 98.40976 89.5916) (width 0.508) (layer F.Cu) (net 2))
 (segment (start 98.298 89.662) (end 98.40976 89.662) (width 0.508) (layer F.Cu) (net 2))
 (segment (start 98.33936 89.662) (end 98.298 89.662) (width 0.508) (layer F.Cu) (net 2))
 (segment (start 98.40976 89.5916) (end 98.33936 89.662) (width 0.508) (layer F.Cu) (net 2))
 (segment (start 98.40976 93.935) (end 98.40396 93.9292) (width 0.508) (layer F.Cu) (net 2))
 (segment (start 98.3996 93.9292) (end 98.40976 93.9292) (width 0.508) (layer F.Cu) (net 2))
 (segment (start 98.40396 93.9292) (end 98.3996 93.9292) (width 0.508) (layer F.Cu) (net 2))
 (segment (start 98.40976 93.935) (end 98.40396 93.9292) (width 0.508) (layer F.Cu) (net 2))
 (segment (start 98.40976 81.20126) (end 98.40976 89.662) (width 1.6256) (layer F.Cu) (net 2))
 (segment (start 98.40976 89.662) (end 98.40976 93.9292) (width 1.6256) (layer F.Cu) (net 2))
 (segment (start 98.40976 93.9292) (end 98.40976 97.25924) (width 1.6256) (layer F.Cu) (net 2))
 (segment (start 98.40976 97.25924) (end 98.409 97.26) (width 1.6256) (layer F.Cu) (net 2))
 (segment (start 103.2002 92.075) (end 103.2002 91.7956) (width 0.508) (layer F.Cu) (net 2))
 (segment (start 102.5906 89.363) (end 102.362 89.5916) (width 0.508) (layer F.Cu) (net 2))
 (segment (start 102.362 89.5916) (end 103.4186 88.535) (width 0.508) (layer F.Cu) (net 2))
 (segment (start 102.5906 91.186) (end 102.5906 89.363) (width 0.508) (layer F.Cu) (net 2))
 (segment (start 103.2002 91.7956) (end 102.5906 91.186) (width 0.508) (layer F.Cu) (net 2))
 (segment (start 90.839 99.97) (end 90.839 79.97092) (width 0.508) (layer B.Cu) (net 7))
 (segment (start 90.839 79.97092) (end 91.70924 79.10068) (width 0.508) (layer B.Cu) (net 7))
 (segment (start 105.6386 91.5416) (end 105.3186 91.2216) (width 0.508) (layer F.Cu) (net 1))
 (segment (start 105.3186 91.2216) (end 105.3186 90.535) (width 0.508) (layer F.Cu) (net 1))
 (segment (start 104.267 92.075) (end 105.3186 91.0234) (width 0.508) (layer F.Cu) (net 1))
 (segment (start 105.3186 91.0234) (end 105.3186 90.535) (width 0.508) (layer F.Cu) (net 1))
 (segment (start 106.934 89.535) (end 105.918 89.535) (width 0.508) (layer B.Cu) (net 3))
 (segment (start 105.6386 86.4616) (end 104.521 86.4616) (width 0.508) (layer F.Cu) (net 3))
 (via (at 104.4956 86.487) (size 0.889) (layers F.Cu B.Cu) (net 3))
 (segment (start 104.521 86.4616) (end 104.4956 86.487) (width 0.508) (layer F.Cu) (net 3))
 (segment (start 105.6386 92.6084) (end 105.2322 92.6084) (width 0.508) (layer F.Cu) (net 3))
 (via (at 104.8766 92.964) (size 0.889) (layers F.Cu B.Cu) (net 3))
 (segment (start 105.2322 92.6084) (end 104.8766 92.964) (width 0.508) (layer F.Cu) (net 3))
 (segment (start 93.90888 97.25988) (end 93.909 97.26) (width 0.508) (layer F.Cu) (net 5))
 (segment (start 93.90888 81.20126) (end 93.90888 97.25988) (width 0.508) (layer F.Cu) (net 5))
 (segment (start 96.40824 81.20126) (end 96.40824 97.25924) (width 1.6256) (layer F.Cu) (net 6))
 (segment (start 96.40824 97.25924) (end 96.409 97.26) (width 1.6256) (layer F.Cu) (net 6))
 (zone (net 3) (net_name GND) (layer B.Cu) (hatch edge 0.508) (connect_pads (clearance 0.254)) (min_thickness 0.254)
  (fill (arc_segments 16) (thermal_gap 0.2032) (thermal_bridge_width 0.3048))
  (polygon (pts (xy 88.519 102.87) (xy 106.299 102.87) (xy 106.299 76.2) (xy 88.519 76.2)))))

